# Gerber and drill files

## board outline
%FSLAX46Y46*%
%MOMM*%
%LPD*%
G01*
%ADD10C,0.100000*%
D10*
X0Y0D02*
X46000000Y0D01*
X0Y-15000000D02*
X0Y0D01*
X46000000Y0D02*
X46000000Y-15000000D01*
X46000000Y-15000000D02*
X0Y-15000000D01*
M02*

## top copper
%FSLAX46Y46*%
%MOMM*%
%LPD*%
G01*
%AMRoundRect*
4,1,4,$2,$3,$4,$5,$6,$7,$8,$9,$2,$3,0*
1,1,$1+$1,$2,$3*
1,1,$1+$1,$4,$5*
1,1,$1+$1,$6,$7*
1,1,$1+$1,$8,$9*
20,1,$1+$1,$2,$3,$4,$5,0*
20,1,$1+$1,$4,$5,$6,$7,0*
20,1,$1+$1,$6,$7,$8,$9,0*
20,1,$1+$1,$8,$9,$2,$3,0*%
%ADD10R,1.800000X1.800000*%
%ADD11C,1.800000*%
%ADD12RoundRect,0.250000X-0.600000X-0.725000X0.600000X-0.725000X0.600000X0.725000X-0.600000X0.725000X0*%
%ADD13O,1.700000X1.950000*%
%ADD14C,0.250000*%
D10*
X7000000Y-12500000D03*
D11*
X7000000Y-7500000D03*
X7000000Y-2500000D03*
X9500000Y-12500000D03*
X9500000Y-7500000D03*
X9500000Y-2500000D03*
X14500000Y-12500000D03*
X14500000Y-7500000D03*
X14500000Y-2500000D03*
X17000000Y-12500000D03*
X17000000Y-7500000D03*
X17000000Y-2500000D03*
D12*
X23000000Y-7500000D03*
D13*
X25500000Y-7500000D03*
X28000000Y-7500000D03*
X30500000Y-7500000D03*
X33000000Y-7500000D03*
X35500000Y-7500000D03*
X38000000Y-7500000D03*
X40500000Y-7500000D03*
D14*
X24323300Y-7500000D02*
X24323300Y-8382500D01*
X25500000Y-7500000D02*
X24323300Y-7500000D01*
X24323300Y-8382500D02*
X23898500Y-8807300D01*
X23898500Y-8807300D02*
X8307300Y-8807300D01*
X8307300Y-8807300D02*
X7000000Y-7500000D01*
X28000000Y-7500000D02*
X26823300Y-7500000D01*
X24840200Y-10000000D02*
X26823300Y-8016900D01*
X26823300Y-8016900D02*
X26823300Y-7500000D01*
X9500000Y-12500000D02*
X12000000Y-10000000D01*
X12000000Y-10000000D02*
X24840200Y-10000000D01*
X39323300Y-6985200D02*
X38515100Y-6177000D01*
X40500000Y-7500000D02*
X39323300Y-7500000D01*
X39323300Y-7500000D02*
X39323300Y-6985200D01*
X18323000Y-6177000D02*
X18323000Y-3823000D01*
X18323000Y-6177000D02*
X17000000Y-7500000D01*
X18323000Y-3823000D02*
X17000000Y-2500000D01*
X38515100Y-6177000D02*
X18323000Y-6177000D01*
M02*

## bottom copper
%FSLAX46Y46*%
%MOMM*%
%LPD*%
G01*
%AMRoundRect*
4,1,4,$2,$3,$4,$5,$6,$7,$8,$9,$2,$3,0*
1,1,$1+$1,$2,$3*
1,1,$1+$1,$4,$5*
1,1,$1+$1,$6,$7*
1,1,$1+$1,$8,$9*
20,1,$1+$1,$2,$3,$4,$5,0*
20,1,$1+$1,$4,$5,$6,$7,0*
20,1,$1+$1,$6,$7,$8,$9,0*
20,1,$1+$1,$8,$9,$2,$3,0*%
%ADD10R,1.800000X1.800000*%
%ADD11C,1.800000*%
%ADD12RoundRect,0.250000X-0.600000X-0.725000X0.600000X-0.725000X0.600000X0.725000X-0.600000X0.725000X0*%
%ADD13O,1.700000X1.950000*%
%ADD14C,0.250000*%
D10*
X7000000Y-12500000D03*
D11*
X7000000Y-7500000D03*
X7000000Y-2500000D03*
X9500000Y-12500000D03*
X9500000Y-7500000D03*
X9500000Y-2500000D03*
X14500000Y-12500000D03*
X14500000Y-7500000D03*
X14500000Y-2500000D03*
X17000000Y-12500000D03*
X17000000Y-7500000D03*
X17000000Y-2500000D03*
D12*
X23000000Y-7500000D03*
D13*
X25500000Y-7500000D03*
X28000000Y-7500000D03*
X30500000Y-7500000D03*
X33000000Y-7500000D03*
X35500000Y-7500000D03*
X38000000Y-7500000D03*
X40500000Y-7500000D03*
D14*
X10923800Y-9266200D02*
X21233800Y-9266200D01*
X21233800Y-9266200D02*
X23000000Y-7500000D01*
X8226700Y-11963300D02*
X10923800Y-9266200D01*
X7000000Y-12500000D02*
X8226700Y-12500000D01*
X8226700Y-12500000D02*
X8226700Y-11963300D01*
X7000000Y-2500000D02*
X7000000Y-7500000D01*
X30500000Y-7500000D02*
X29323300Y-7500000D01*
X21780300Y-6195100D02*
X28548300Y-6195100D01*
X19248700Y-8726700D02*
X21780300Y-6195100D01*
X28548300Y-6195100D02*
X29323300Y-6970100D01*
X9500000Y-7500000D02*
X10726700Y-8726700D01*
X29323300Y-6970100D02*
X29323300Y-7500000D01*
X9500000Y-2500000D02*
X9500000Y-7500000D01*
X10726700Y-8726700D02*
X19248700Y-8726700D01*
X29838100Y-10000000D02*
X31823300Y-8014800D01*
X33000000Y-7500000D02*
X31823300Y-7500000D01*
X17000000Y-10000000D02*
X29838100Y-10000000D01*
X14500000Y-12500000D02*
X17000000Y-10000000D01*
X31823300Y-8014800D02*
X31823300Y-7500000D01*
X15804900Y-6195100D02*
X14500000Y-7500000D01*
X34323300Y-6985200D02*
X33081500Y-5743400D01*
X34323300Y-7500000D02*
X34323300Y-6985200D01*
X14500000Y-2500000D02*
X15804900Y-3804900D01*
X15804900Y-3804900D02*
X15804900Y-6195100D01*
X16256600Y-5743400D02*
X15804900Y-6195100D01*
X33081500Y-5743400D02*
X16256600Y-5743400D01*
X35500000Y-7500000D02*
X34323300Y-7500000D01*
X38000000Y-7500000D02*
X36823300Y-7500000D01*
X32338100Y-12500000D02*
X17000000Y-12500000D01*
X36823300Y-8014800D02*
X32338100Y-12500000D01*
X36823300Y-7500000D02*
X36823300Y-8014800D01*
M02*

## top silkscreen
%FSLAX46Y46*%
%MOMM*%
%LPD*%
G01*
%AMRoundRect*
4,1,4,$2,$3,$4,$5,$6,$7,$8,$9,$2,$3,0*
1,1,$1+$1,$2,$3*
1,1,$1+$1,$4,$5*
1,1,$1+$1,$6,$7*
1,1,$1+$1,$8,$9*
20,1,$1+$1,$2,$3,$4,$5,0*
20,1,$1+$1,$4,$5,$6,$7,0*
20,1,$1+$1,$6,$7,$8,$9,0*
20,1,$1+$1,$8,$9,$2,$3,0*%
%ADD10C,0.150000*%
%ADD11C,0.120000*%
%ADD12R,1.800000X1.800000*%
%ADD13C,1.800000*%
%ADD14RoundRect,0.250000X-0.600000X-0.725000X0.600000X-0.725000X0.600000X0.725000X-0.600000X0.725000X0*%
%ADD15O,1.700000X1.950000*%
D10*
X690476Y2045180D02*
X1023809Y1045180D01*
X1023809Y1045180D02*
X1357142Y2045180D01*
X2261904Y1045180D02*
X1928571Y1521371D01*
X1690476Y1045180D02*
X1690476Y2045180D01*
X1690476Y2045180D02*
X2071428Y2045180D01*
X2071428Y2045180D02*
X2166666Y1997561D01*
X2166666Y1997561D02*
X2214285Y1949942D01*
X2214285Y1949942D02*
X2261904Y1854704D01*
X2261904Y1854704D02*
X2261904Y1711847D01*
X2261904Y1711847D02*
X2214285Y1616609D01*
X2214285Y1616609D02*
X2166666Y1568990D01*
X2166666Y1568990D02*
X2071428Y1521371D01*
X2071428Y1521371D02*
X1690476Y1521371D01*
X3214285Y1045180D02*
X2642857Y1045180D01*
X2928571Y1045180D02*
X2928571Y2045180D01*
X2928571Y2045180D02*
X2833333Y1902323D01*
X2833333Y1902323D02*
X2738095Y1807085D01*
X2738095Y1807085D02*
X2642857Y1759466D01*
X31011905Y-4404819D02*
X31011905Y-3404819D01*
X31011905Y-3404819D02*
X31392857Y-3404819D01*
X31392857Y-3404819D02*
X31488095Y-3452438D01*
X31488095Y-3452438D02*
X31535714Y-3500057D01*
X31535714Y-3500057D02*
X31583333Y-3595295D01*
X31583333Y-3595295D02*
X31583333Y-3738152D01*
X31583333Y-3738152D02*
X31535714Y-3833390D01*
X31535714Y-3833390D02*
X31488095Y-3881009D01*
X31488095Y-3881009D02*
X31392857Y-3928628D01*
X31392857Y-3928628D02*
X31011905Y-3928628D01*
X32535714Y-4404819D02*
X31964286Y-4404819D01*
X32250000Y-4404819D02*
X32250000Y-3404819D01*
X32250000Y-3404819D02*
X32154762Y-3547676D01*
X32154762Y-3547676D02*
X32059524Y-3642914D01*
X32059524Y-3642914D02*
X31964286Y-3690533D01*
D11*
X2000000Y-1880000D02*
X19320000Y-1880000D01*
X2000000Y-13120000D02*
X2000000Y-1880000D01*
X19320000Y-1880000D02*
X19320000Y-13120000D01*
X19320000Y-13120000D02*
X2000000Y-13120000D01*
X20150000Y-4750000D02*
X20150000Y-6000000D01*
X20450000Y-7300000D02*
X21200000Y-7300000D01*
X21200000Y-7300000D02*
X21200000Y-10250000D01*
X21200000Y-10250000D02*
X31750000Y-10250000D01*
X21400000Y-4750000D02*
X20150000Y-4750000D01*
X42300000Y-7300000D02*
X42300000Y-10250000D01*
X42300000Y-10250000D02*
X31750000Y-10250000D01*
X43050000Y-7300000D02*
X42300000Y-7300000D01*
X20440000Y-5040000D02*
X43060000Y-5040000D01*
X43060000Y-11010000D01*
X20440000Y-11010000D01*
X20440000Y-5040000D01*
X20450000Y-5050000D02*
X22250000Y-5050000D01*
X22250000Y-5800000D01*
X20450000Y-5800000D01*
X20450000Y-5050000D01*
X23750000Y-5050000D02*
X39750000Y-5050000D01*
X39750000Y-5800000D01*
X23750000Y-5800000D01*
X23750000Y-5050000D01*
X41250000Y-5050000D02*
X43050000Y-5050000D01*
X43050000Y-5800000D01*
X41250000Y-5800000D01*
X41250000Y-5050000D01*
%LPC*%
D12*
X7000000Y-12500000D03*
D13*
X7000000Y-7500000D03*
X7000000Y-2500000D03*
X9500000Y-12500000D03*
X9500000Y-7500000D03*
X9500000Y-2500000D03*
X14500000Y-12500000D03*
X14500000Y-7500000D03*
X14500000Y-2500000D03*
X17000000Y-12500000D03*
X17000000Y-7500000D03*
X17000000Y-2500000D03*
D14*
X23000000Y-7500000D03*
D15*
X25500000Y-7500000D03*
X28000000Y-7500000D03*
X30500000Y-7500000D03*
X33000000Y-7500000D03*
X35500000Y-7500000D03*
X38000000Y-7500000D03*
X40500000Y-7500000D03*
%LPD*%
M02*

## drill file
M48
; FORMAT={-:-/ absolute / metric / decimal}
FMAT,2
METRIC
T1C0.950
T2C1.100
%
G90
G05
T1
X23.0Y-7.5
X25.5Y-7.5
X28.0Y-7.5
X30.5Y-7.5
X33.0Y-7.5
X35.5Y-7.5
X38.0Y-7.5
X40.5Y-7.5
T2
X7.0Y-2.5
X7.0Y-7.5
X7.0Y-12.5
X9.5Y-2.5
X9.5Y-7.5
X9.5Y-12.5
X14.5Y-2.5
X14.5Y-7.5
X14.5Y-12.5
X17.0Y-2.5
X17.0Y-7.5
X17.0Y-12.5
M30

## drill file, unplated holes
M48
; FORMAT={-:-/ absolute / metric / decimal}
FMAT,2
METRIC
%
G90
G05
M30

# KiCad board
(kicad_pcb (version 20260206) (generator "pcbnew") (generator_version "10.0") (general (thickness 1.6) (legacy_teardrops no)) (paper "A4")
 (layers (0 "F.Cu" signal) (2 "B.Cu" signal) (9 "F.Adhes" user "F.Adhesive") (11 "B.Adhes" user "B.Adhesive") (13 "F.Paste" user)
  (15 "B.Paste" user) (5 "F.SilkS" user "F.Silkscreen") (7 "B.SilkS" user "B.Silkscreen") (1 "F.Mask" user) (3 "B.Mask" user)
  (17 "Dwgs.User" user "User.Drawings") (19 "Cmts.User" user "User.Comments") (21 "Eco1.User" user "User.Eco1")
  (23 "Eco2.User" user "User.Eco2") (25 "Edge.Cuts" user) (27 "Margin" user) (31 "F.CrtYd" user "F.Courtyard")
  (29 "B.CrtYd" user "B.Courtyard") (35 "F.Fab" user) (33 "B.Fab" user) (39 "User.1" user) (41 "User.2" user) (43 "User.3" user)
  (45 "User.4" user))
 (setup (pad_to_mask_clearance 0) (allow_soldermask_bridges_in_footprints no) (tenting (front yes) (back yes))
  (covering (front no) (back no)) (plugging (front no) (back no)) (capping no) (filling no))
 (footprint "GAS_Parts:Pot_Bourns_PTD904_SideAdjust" (layer "F.Cu") (at 2 7.5)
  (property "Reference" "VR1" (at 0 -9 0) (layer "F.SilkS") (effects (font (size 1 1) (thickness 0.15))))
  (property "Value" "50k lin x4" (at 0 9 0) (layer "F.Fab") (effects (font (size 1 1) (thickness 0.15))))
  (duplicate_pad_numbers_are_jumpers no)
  (fp_line (start 0 -5.62) (end 17.32 -5.62) (stroke (width 0.12) (type solid)) (layer "F.SilkS"))
  (fp_line (start 0 5.62) (end 0 -5.62) (stroke (width 0.12) (type solid)) (layer "F.SilkS"))
  (fp_line (start 17.32 -5.62) (end 17.32 5.62) (stroke (width 0.12) (type solid)) (layer "F.SilkS"))
  (fp_line (start 17.32 5.62) (end 0 5.62) (stroke (width 0.12) (type solid)) (layer "F.SilkS"))
  (pad "11" thru_hole rect (at 5 5) (size 1.8 1.8) (drill 1.1) (layers "*.Cu" "*.Mask") (remove_unused_layers no) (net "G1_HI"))
  (pad "12" thru_hole circle (at 5 0) (size 1.8 1.8) (drill 1.1) (layers "*.Cu" "*.Mask") (remove_unused_layers no) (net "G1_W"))
  (pad "13" thru_hole circle (at 5 -5) (size 1.8 1.8) (drill 1.1) (layers "*.Cu" "*.Mask") (remove_unused_layers no) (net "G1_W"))
  (pad "21" thru_hole circle (at 7.5 5) (size 1.8 1.8) (drill 1.1) (layers "*.Cu" "*.Mask") (remove_unused_layers no) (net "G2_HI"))
  (pad "22" thru_hole circle (at 7.5 0) (size 1.8 1.8) (drill 1.1) (layers "*.Cu" "*.Mask") (remove_unused_layers no) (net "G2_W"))
  (pad "23" thru_hole circle (at 7.5 -5) (size 1.8 1.8) (drill 1.1) (layers "*.Cu" "*.Mask") (remove_unused_layers no) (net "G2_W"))
  (pad "31" thru_hole circle (at 12.5 5) (size 1.8 1.8) (drill 1.1) (layers "*.Cu" "*.Mask") (remove_unused_layers no) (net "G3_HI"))
  (pad "32" thru_hole circle (at 12.5 0) (size 1.8 1.8) (drill 1.1) (layers "*.Cu" "*.Mask") (remove_unused_layers no) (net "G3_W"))
  (pad "33" thru_hole circle (at 12.5 -5) (size 1.8 1.8) (drill 1.1) (layers "*.Cu" "*.Mask") (remove_unused_layers no) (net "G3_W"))
  (pad "41" thru_hole circle (at 15 5) (size 1.8 1.8) (drill 1.1) (layers "*.Cu" "*.Mask") (remove_unused_layers no) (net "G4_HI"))
  (pad "42" thru_hole circle (at 15 0) (size 1.8 1.8) (drill 1.1) (layers "*.Cu" "*.Mask") (remove_unused_layers no) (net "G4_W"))
  (pad "43" thru_hole circle (at 15 -5) (size 1.8 1.8) (drill 1.1) (layers "*.Cu" "*.Mask") (remove_unused_layers no) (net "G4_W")))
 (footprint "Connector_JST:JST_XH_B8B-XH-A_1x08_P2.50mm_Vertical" (layer "F.Cu") (at 23 7.5)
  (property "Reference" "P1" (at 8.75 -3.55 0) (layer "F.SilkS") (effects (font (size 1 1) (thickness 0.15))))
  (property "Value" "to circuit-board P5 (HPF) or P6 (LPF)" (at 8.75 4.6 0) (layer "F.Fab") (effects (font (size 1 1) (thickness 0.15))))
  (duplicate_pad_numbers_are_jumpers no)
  (fp_line (start -2.85 -2.75) (end -2.85 -1.5) (stroke (width 0.12) (type solid)) (layer "F.SilkS"))
  (fp_line (start -2.55 -0.2) (end -1.8 -0.2) (stroke (width 0.12) (type solid)) (layer "F.SilkS"))
  (fp_line (start -1.8 -0.2) (end -1.8 2.75) (stroke (width 0.12) (type solid)) (layer "F.SilkS"))
  (fp_line (start -1.8 2.75) (end 8.75 2.75) (stroke (width 0.12) (type solid)) (layer "F.SilkS"))
  (fp_line (start -1.6 -2.75) (end -2.85 -2.75) (stroke (width 0.12) (type solid)) (layer "F.SilkS"))
  (fp_line (start 19.3 -0.2) (end 19.3 2.75) (stroke (width 0.12) (type solid)) (layer "F.SilkS"))
  (fp_line (start 19.3 2.75) (end 8.75 2.75) (stroke (width 0.12) (type solid)) (layer "F.SilkS"))
  (fp_line (start 20.05 -0.2) (end 19.3 -0.2) (stroke (width 0.12) (type solid)) (layer "F.SilkS"))
  (fp_rect (start -2.56 -2.46) (end 20.06 3.51) (stroke (width 0.12) (type solid)) (fill no) (layer "F.SilkS"))
  (fp_rect (start -2.55 -2.45) (end -0.75 -1.7) (stroke (width 0.12) (type solid)) (fill no) (layer "F.SilkS"))
  (fp_rect (start 0.75 -2.45) (end 16.75 -1.7) (stroke (width 0.12) (type solid)) (fill no) (layer "F.SilkS"))
  (fp_rect (start 18.25 -2.45) (end 20.05 -1.7) (stroke (width 0.12) (type solid)) (fill no) (layer "F.SilkS"))
  (pad "1" thru_hole roundrect (at 0 0) (size 1.7 1.95) (drill 0.95) (layers "*.Cu" "*.Mask") (remove_unused_layers no)
   (roundrect_rratio 0.147059) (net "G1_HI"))
  (pad "2" thru_hole oval (at 2.5 0) (size 1.7 1.95) (drill 0.95) (layers "*.Cu" "*.Mask") (remove_unused_layers no) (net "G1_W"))
  (pad "3" thru_hole oval (at 5 0) (size 1.7 1.95) (drill 0.95) (layers "*.Cu" "*.Mask") (remove_unused_layers no) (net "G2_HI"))
  (pad "4" thru_hole oval (at 7.5 0) (size 1.7 1.95) (drill 0.95) (layers "*.Cu" "*.Mask") (remove_unused_layers no) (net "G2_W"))
  (pad "5" thru_hole oval (at 10 0) (size 1.7 1.95) (drill 0.95) (layers "*.Cu" "*.Mask") (remove_unused_layers no) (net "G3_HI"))
  (pad "6" thru_hole oval (at 12.5 0) (size 1.7 1.95) (drill 0.95) (layers "*.Cu" "*.Mask") (remove_unused_layers no) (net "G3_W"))
  (pad "7" thru_hole oval (at 15 0) (size 1.7 1.95) (drill 0.95) (layers "*.Cu" "*.Mask") (remove_unused_layers no) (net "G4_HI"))
  (pad "8" thru_hole oval (at 17.5 0) (size 1.7 1.95) (drill 0.95) (layers "*.Cu" "*.Mask") (remove_unused_layers no) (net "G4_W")))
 (gr_line (start 0 0) (end 46 0) (stroke (width 0.1) (type default)) (layer "Edge.Cuts"))
 (gr_line (start 0 15) (end 0 0) (stroke (width 0.1) (type default)) (layer "Edge.Cuts"))
 (gr_line (start 46 0) (end 46 15) (stroke (width 0.1) (type default)) (layer "Edge.Cuts"))
 (gr_line (start 46 15) (end 0 15) (stroke (width 0.1) (type default)) (layer "Edge.Cuts"))
 (segment (start 10.9238 9.2662) (end 21.2338 9.2662) (width 0.25) (layer "B.Cu") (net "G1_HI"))
 (segment (start 21.2338 9.2662) (end 23 7.5) (width 0.25) (layer "B.Cu") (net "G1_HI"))
 (segment (start 8.2267 11.9633) (end 10.9238 9.2662) (width 0.25) (layer "B.Cu") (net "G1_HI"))
 (segment (start 7 12.5) (end 8.2267 12.5) (width 0.25) (layer "B.Cu") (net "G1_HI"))
 (segment (start 8.2267 12.5) (end 8.2267 11.9633) (width 0.25) (layer "B.Cu") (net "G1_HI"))
 (segment (start 24.3233 7.5) (end 24.3233 8.3825) (width 0.25) (layer "F.Cu") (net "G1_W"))
 (segment (start 25.5 7.5) (end 24.3233 7.5) (width 0.25) (layer "F.Cu") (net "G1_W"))
 (segment (start 24.3233 8.3825) (end 23.8985 8.8073) (width 0.25) (layer "F.Cu") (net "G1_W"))
 (segment (start 23.8985 8.8073) (end 8.3073 8.8073) (width 0.25) (layer "F.Cu") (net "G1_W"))
 (segment (start 8.3073 8.8073) (end 7 7.5) (width 0.25) (layer "F.Cu") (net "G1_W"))
 (segment (start 7 2.5) (end 7 7.5) (width 0.25) (layer "B.Cu") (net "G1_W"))
 (segment (start 28 7.5) (end 26.8233 7.5) (width 0.25) (layer "F.Cu") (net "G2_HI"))
 (segment (start 24.8402 10) (end 26.8233 8.0169) (width 0.25) (layer "F.Cu") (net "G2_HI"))
 (segment (start 26.8233 8.0169) (end 26.8233 7.5) (width 0.25) (layer "F.Cu") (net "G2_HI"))
 (segment (start 9.5 12.5) (end 12 10) (width 0.25) (layer "F.Cu") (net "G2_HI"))
 (segment (start 12 10) (end 24.8402 10) (width 0.25) (layer "F.Cu") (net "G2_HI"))
 (segment (start 30.5 7.5) (end 29.3233 7.5) (width 0.25) (layer "B.Cu") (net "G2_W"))
 (segment (start 21.7803 6.1951) (end 28.5483 6.1951) (width 0.25) (layer "B.Cu") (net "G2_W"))
 (segment (start 19.2487 8.7267) (end 21.7803 6.1951) (width 0.25) (layer "B.Cu") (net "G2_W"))
 (segment (start 28.5483 6.1951) (end 29.3233 6.9701) (width 0.25) (layer "B.Cu") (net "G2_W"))
 (segment (start 9.5 7.5) (end 10.7267 8.7267) (width 0.25) (layer "B.Cu") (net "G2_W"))
 (segment (start 29.3233 6.9701) (end 29.3233 7.5) (width 0.25) (layer "B.Cu") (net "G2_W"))
 (segment (start 9.5 2.5) (end 9.5 7.5) (width 0.25) (layer "B.Cu") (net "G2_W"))
 (segment (start 10.7267 8.7267) (end 19.2487 8.7267) (width 0.25) (layer "B.Cu") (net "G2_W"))
 (segment (start 29.8381 10) (end 31.8233 8.0148) (width 0.25) (layer "B.Cu") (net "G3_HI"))
 (segment (start 33 7.5) (end 31.8233 7.5) (width 0.25) (layer "B.Cu") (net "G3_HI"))
 (segment (start 17 10) (end 29.8381 10) (width 0.25) (layer "B.Cu") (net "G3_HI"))
 (segment (start 14.5 12.5) (end 17 10) (width 0.25) (layer "B.Cu") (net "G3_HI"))
 (segment (start 31.8233 8.0148) (end 31.8233 7.5) (width 0.25) (layer "B.Cu") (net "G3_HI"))
 (segment (start 15.8049 6.1951) (end 14.5 7.5) (width 0.25) (layer "B.Cu") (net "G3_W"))
 (segment (start 34.3233 6.9852) (end 33.0815 5.7434) (width 0.25) (layer "B.Cu") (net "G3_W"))
 (segment (start 34.3233 7.5) (end 34.3233 6.9852) (width 0.25) (layer "B.Cu") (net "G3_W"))
 (segment (start 14.5 2.5) (end 15.8049 3.8049) (width 0.25) (layer "B.Cu") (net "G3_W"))
 (segment (start 15.8049 3.8049) (end 15.8049 6.1951) (width 0.25) (layer "B.Cu") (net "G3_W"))
 (segment (start 16.2566 5.7434) (end 15.8049 6.1951) (width 0.25) (layer "B.Cu") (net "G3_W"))
 (segment (start 33.0815 5.7434) (end 16.2566 5.7434) (width 0.25) (layer "B.Cu") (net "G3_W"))
 (segment (start 35.5 7.5) (end 34.3233 7.5) (width 0.25) (layer "B.Cu") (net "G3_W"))
 (segment (start 38 7.5) (end 36.8233 7.5) (width 0.25) (layer "B.Cu") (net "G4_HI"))
 (segment (start 32.3381 12.5) (end 17 12.5) (width 0.25) (layer "B.Cu") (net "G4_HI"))
 (segment (start 36.8233 8.0148) (end 32.3381 12.5) (width 0.25) (layer "B.Cu") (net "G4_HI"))
 (segment (start 36.8233 7.5) (end 36.8233 8.0148) (width 0.25) (layer "B.Cu") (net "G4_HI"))
 (segment (start 39.3233 6.9852) (end 38.5151 6.177) (width 0.25) (layer "F.Cu") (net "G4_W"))
 (segment (start 40.5 7.5) (end 39.3233 7.5) (width 0.25) (layer "F.Cu") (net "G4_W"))
 (segment (start 39.3233 7.5) (end 39.3233 6.9852) (width 0.25) (layer "F.Cu") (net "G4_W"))
 (segment (start 18.323 6.177) (end 18.323 3.823) (width 0.25) (layer "F.Cu") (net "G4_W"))
 (segment (start 18.323 6.177) (end 17 7.5) (width 0.25) (layer "F.Cu") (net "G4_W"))
 (segment (start 18.323 3.823) (end 17 2.5) (width 0.25) (layer "F.Cu") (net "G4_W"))
 (segment (start 38.5151 6.177) (end 18.323 6.177) (width 0.25) (layer "F.Cu") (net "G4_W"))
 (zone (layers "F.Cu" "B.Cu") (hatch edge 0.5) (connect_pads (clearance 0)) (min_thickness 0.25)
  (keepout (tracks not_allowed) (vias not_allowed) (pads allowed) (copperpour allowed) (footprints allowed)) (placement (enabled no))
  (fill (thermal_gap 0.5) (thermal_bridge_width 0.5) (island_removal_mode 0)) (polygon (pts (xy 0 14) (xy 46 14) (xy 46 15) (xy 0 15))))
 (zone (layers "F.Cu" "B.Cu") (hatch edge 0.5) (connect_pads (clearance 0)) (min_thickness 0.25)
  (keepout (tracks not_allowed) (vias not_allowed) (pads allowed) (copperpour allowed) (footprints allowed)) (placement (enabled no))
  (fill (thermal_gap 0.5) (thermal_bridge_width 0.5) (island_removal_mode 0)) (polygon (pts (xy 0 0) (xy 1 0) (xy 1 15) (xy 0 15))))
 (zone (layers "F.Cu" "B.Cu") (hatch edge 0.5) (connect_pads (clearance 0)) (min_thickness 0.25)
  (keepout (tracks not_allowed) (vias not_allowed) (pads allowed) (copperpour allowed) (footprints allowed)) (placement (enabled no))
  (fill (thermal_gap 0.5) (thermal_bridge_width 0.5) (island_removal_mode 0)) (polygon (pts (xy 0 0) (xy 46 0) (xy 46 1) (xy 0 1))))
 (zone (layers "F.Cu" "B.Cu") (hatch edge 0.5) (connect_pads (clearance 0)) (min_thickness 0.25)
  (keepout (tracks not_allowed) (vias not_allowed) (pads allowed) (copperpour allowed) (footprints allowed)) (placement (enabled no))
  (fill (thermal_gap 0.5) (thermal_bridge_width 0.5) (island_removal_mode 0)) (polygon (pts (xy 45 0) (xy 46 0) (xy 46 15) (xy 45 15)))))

